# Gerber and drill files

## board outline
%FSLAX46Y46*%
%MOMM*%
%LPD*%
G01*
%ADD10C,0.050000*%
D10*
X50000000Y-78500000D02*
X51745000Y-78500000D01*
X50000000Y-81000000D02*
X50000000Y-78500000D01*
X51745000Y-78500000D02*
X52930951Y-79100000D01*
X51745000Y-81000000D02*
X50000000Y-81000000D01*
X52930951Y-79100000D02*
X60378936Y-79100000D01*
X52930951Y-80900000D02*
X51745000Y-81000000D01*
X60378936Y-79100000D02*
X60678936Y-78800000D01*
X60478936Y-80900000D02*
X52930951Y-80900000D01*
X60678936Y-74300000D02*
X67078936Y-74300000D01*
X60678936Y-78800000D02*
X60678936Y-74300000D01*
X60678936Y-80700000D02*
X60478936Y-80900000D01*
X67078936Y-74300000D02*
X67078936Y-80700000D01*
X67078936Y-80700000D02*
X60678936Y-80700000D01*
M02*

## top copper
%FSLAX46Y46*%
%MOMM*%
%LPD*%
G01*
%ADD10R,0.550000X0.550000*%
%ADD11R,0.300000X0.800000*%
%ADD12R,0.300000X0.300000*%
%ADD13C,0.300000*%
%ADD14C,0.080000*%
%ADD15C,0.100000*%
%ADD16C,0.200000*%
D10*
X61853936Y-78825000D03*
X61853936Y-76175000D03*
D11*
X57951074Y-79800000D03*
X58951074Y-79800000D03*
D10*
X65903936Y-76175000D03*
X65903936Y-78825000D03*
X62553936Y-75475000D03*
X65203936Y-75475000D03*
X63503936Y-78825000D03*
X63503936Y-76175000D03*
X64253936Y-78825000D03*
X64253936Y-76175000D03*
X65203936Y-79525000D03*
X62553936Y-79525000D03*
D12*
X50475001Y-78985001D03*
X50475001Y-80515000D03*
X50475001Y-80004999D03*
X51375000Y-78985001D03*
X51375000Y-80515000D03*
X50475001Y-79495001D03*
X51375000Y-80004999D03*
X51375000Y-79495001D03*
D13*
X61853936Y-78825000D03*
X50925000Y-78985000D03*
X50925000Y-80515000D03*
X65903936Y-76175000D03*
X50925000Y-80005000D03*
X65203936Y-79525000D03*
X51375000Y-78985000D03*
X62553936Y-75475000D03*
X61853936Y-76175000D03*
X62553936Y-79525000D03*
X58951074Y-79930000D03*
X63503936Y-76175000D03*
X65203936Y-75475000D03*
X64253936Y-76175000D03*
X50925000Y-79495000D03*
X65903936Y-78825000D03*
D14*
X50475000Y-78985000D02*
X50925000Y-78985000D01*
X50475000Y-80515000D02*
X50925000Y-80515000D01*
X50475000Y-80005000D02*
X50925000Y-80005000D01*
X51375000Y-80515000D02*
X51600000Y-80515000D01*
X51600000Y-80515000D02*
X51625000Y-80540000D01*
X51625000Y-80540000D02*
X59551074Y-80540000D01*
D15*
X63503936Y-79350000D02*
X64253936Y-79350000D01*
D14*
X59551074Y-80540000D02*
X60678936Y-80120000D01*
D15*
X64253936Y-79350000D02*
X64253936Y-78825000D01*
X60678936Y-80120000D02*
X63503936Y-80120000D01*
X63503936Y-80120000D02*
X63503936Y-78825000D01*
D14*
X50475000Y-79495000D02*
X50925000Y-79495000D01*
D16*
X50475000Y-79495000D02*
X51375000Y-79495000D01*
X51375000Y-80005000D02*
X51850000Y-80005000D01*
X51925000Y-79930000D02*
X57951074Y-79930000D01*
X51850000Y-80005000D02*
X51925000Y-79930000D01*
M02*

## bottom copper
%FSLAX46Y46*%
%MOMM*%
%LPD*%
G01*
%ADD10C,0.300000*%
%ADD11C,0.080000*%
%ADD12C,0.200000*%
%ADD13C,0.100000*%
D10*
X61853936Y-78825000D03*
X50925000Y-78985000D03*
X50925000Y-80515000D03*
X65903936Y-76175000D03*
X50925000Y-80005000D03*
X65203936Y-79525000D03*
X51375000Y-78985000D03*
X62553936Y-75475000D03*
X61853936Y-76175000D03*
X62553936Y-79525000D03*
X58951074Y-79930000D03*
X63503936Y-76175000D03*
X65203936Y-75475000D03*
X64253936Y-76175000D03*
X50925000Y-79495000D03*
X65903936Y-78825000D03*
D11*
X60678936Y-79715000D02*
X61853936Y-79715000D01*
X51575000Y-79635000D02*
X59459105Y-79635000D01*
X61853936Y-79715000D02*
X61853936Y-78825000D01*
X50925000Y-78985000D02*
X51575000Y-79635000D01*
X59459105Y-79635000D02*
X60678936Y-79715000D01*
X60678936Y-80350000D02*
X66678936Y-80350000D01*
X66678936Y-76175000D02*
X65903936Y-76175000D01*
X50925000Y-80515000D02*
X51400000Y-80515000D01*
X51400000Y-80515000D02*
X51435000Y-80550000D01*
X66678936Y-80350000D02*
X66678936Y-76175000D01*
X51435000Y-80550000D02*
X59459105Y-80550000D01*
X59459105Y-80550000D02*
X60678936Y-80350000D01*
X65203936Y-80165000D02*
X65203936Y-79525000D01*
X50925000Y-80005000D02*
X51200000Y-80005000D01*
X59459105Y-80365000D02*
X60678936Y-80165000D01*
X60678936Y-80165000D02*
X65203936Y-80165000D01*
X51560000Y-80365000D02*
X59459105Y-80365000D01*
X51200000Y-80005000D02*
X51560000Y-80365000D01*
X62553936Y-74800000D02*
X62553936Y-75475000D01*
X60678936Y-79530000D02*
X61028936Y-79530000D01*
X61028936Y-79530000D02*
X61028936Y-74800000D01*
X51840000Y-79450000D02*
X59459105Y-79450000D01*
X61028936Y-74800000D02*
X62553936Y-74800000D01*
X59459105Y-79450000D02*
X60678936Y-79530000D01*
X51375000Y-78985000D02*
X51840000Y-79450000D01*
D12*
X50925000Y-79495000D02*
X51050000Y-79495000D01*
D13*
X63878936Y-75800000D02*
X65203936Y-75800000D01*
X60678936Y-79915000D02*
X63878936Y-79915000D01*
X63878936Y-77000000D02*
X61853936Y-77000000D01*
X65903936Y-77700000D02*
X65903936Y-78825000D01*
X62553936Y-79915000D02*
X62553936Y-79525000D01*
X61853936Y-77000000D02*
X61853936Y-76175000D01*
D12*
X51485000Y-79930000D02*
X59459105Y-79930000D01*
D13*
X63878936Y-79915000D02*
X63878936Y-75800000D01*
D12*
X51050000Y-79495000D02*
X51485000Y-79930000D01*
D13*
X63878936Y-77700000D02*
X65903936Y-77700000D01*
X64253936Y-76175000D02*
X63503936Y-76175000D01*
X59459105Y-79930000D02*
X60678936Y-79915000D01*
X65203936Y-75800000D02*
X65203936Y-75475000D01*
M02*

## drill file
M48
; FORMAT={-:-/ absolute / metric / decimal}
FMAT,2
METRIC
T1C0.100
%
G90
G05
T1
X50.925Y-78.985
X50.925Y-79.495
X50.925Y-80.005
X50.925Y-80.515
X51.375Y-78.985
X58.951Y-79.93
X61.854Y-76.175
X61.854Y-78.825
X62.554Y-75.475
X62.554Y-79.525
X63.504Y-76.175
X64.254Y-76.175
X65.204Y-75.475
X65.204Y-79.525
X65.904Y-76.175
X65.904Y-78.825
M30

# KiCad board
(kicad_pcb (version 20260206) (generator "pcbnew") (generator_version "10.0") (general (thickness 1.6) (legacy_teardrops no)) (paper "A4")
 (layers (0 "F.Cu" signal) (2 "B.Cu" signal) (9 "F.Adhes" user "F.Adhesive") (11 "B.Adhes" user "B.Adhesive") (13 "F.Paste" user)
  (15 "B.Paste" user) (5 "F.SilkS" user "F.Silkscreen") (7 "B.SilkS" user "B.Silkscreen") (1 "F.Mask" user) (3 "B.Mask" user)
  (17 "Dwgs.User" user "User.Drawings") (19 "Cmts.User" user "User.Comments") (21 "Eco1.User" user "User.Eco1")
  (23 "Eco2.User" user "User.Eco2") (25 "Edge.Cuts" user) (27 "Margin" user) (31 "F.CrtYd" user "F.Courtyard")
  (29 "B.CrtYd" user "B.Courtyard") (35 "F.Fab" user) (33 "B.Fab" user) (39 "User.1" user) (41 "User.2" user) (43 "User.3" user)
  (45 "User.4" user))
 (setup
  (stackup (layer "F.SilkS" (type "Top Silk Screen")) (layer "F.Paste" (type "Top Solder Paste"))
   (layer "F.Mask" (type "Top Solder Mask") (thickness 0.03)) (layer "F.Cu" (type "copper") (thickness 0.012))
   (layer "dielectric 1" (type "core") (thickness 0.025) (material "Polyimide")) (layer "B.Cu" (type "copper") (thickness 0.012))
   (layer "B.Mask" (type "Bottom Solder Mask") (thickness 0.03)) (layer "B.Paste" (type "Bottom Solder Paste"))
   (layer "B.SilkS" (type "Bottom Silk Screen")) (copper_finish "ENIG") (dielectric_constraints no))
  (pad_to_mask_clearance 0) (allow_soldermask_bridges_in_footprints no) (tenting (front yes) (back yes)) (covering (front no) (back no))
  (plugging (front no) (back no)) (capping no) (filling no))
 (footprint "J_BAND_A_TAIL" (layer "F.Cu") (at 50.9 79.75)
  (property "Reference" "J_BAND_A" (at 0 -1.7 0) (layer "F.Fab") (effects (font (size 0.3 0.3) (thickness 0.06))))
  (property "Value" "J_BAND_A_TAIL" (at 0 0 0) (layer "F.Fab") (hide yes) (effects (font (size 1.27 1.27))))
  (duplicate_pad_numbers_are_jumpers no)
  (pad "1" smd rect (at -0.424999 -0.764999) (size 0.3 0.3) (layers "F.Cu" "F.Mask") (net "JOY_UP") (solder_mask_margin 0.05)
   (thermal_bridge_angle 45))
  (pad "2" smd rect (at -0.424999 0.765) (size 0.3 0.3) (layers "F.Cu" "F.Mask") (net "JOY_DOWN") (solder_mask_margin 0.05)
   (thermal_bridge_angle 45))
  (pad "3" smd rect (at -0.424999 0.254999) (size 0.3 0.3) (layers "F.Cu" "F.Mask") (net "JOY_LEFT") (solder_mask_margin 0.05)
   (thermal_bridge_angle 45))
  (pad "4" smd rect (at 0.475 -0.764999) (size 0.3 0.3) (layers "F.Cu" "F.Mask") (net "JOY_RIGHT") (solder_mask_margin 0.05)
   (thermal_bridge_angle 45))
  (pad "5" smd rect (at 0.475 0.765) (size 0.3 0.3) (layers "F.Cu" "F.Mask") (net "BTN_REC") (solder_mask_margin 0.05)
   (thermal_bridge_angle 45))
  (pad "6" smd rect (at -0.424999 -0.254999) (size 0.3 0.3) (layers "F.Cu" "F.Mask") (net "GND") (solder_mask_margin 0.05)
   (thermal_bridge_angle 45))
  (pad "7" smd rect (at 0.475 0.254999) (size 0.3 0.3) (layers "F.Cu" "F.Mask") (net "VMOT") (solder_mask_margin 0.05)
   (thermal_bridge_angle 45))
  (pad "8" smd rect (at 0.475 -0.254999) (size 0.3 0.3) (layers "F.Cu" "F.Mask") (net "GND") (solder_mask_margin 0.05)
   (thermal_bridge_angle 45)))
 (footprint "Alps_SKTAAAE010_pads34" (layer "F.Cu") (at 61.478936 77.5 90)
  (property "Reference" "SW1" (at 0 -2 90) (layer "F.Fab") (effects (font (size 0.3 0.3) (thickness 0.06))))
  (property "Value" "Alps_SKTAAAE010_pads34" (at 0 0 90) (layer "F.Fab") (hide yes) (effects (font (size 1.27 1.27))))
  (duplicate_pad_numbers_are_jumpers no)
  (pad "3" smd rect (at -1.325 0.375 90) (size 0.55 0.55) (layers "F.Cu" "F.Mask" "F.Paste") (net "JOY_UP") (solder_mask_margin 0.05)
   (thermal_bridge_angle 45))
  (pad "4" smd rect (at 1.325 0.375 90) (size 0.55 0.55) (layers "F.Cu" "F.Mask" "F.Paste") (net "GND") (solder_mask_margin 0.05)
   (thermal_bridge_angle 45)))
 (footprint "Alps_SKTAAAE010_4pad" (layer "F.Cu") (at 63.878936 77.5 90)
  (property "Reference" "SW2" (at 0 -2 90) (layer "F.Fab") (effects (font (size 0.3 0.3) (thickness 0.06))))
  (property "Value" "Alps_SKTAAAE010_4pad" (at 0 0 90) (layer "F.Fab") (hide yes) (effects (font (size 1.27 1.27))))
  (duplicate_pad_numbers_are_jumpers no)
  (pad "1" smd rect (at -1.325 -0.375 90) (size 0.55 0.55) (layers "F.Cu" "F.Mask" "F.Paste") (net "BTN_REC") (solder_mask_margin 0.05)
   (thermal_bridge_angle 45))
  (pad "2" smd rect (at 1.325 -0.375 90) (size 0.55 0.55) (layers "F.Cu" "F.Mask" "F.Paste") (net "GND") (solder_mask_margin 0.05)
   (thermal_bridge_angle 45))
  (pad "3" smd rect (at -1.325 0.375 90) (size 0.55 0.55) (layers "F.Cu" "F.Mask" "F.Paste") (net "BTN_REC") (solder_mask_margin 0.05)
   (thermal_bridge_angle 45))
  (pad "4" smd rect (at 1.325 0.375 90) (size 0.55 0.55) (layers "F.Cu" "F.Mask" "F.Paste") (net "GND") (solder_mask_margin 0.05)
   (thermal_bridge_angle 45)))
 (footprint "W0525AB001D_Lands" (layer "F.Cu") (at 58.451074 79.93)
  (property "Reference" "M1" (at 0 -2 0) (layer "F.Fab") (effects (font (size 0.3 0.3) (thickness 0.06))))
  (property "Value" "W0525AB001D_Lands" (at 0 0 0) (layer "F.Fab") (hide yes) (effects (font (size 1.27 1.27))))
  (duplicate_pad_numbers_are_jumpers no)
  (pad "1" smd rect (at -0.5 -0.13) (size 0.3 0.8) (layers "F.Cu" "F.Mask") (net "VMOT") (solder_mask_margin 0.05) (thermal_bridge_angle 45))
  (pad "2" smd rect (at 0.5 -0.13) (size 0.3 0.8) (layers "F.Cu" "F.Mask") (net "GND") (solder_mask_margin 0.05) (thermal_bridge_angle 45)))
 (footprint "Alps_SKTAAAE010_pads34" (layer "F.Cu") (at 66.278936 77.5 -90)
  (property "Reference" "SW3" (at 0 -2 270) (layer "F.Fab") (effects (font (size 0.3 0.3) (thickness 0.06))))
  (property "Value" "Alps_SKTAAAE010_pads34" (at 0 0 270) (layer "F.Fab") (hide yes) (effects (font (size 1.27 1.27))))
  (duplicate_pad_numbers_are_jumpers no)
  (pad "3" smd rect (at -1.325 0.375 270) (size 0.55 0.55) (layers "F.Cu" "F.Mask" "F.Paste") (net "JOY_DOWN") (solder_mask_margin 0.05)
   (thermal_bridge_angle 45))
  (pad "4" smd rect (at 1.325 0.375 270) (size 0.55 0.55) (layers "F.Cu" "F.Mask" "F.Paste") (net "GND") (solder_mask_margin 0.05)
   (thermal_bridge_angle 45)))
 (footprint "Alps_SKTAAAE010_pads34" (layer "F.Cu") (at 63.878936 79.9 180)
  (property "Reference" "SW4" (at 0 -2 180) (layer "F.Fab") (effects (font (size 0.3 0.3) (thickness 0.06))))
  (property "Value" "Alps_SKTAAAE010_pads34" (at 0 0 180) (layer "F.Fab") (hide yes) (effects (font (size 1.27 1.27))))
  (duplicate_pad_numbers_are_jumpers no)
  (pad "3" smd rect (at -1.325 0.375 180) (size 0.55 0.55) (layers "F.Cu" "F.Mask" "F.Paste") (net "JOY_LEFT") (solder_mask_margin 0.05)
   (thermal_bridge_angle 45))
  (pad "4" smd rect (at 1.325 0.375 180) (size 0.55 0.55) (layers "F.Cu" "F.Mask" "F.Paste") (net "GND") (solder_mask_margin 0.05)
   (thermal_bridge_angle 45)))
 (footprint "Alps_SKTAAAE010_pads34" (layer "F.Cu") (at 63.878936 75.1)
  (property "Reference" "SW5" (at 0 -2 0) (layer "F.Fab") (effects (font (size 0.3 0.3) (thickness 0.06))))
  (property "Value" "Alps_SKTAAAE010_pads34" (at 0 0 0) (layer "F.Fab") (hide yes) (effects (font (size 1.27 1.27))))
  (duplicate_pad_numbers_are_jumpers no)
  (pad "3" smd rect (at -1.325 0.375) (size 0.55 0.55) (layers "F.Cu" "F.Mask" "F.Paste") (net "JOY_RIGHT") (solder_mask_margin 0.05)
   (thermal_bridge_angle 45))
  (pad "4" smd rect (at 1.325 0.375) (size 0.55 0.55) (layers "F.Cu" "F.Mask" "F.Paste") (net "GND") (solder_mask_margin 0.05)
   (thermal_bridge_angle 45)))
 (gr_line (start 50 78.5) (end 51.745 78.5) (stroke (width 0.05) (type default)) (layer "Edge.Cuts"))
 (gr_line (start 50 81) (end 50 78.5) (stroke (width 0.05) (type default)) (layer "Edge.Cuts"))
 (gr_line (start 51.745 78.5) (end 52.930951 79.1) (stroke (width 0.05) (type default)) (layer "Edge.Cuts"))
 (gr_line (start 51.745 81) (end 50 81) (stroke (width 0.05) (type default)) (layer "Edge.Cuts"))
 (gr_line (start 52.930951 79.1) (end 60.378936 79.1) (stroke (width 0.05) (type default)) (layer "Edge.Cuts"))
 (gr_line (start 52.930951 80.9) (end 51.745 81) (stroke (width 0.05) (type default)) (layer "Edge.Cuts"))
 (gr_line (start 60.378936 79.1) (end 60.678936 78.8) (stroke (width 0.05) (type default)) (layer "Edge.Cuts"))
 (gr_line (start 60.478936 80.9) (end 52.930951 80.9) (stroke (width 0.05) (type default)) (layer "Edge.Cuts"))
 (gr_line (start 60.678936 74.3) (end 67.078936 74.3) (stroke (width 0.05) (type default)) (layer "Edge.Cuts"))
 (gr_line (start 60.678936 78.8) (end 60.678936 74.3) (stroke (width 0.05) (type default)) (layer "Edge.Cuts"))
 (gr_line (start 60.678936 80.7) (end 60.478936 80.9) (stroke (width 0.05) (type default)) (layer "Edge.Cuts"))
 (gr_line (start 67.078936 74.3) (end 67.078936 80.7) (stroke (width 0.05) (type default)) (layer "Edge.Cuts"))
 (gr_line (start 67.078936 80.7) (end 60.678936 80.7) (stroke (width 0.05) (type default)) (layer "Edge.Cuts"))
 (segment (start 50.475 78.985) (end 50.925 78.985) (width 0.08) (layer "F.Cu") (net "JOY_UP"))
 (via (at 61.853936 78.825) (size 0.3) (drill 0.1) (layers "F.Cu" "B.Cu") (tenting (front yes) (back yes)) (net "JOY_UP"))
 (via (at 50.925 78.985) (size 0.3) (drill 0.1) (layers "F.Cu" "B.Cu") (tenting (front yes) (back yes)) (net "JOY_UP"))
 (segment (start 60.678936 79.715) (end 61.853936 79.715) (width 0.08) (layer "B.Cu") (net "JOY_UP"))
 (segment (start 61.853936 79.715) (end 61.853936 78.825) (width 0.08) (layer "B.Cu") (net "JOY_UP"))
 (segment (start 59.459105 79.635) (end 60.678936 79.715) (width 0.08) (layer "B.Cu") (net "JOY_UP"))
 (segment (start 51.575 79.635) (end 59.459105 79.635) (width 0.08) (layer "B.Cu") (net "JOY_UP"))
 (segment (start 50.925 78.985) (end 51.575 79.635) (width 0.08) (layer "B.Cu") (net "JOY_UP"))
 (segment (start 50.475 80.515) (end 50.925 80.515) (width 0.08) (layer "F.Cu") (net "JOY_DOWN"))
 (via (at 50.925 80.515) (size 0.3) (drill 0.1) (layers "F.Cu" "B.Cu") (tenting (front yes) (back yes)) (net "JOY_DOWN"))
 (via (at 65.903936 76.175) (size 0.3) (drill 0.1) (layers "F.Cu" "B.Cu") (tenting (front yes) (back yes)) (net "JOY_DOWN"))
 (segment (start 66.678936 80.35) (end 66.678936 76.175) (width 0.08) (layer "B.Cu") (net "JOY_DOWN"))
 (segment (start 66.678936 76.175) (end 65.903936 76.175) (width 0.08) (layer "B.Cu") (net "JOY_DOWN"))
 (segment (start 60.678936 80.35) (end 66.678936 80.35) (width 0.08) (layer "B.Cu") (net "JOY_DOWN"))
 (segment (start 59.459105 80.55) (end 60.678936 80.35) (width 0.08) (layer "B.Cu") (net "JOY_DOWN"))
 (segment (start 51.435 80.55) (end 59.459105 80.55) (width 0.08) (layer "B.Cu") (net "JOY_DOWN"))
 (segment (start 51.4 80.515) (end 51.435 80.55) (width 0.08) (layer "B.Cu") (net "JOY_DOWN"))
 (segment (start 50.925 80.515) (end 51.4 80.515) (width 0.08) (layer "B.Cu") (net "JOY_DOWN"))
 (segment (start 50.475 80.005) (end 50.925 80.005) (width 0.08) (layer "F.Cu") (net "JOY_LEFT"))
 (via (at 65.203936 79.525) (size 0.3) (drill 0.1) (layers "F.Cu" "B.Cu") (tenting (front yes) (back yes)) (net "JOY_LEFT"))
 (via (at 50.925 80.005) (size 0.3) (drill 0.1) (layers "F.Cu" "B.Cu") (tenting (front yes) (back yes)) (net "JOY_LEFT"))
 (segment (start 51.56 80.365) (end 59.459105 80.365) (width 0.08) (layer "B.Cu") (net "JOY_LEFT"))
 (segment (start 65.203936 80.165) (end 65.203936 79.525) (width 0.08) (layer "B.Cu") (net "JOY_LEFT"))
 (segment (start 60.678936 80.165) (end 65.203936 80.165) (width 0.08) (layer "B.Cu") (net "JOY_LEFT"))
 (segment (start 59.459105 80.365) (end 60.678936 80.165) (width 0.08) (layer "B.Cu") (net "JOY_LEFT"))
 (segment (start 51.2 80.005) (end 51.56 80.365) (width 0.08) (layer "B.Cu") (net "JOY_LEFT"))
 (segment (start 50.925 80.005) (end 51.2 80.005) (width 0.08) (layer "B.Cu") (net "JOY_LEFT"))
 (via (at 51.375 78.985) (size 0.3) (drill 0.1) (layers "F.Cu" "B.Cu") (tenting (front yes) (back yes)) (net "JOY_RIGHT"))
 (via (at 62.553936 75.475) (size 0.3) (drill 0.1) (layers "F.Cu" "B.Cu") (tenting (front yes) (back yes)) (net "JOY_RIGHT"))
 (segment (start 51.375 78.985) (end 51.84 79.45) (width 0.08) (layer "B.Cu") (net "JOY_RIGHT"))
 (segment (start 62.553936 74.8) (end 62.553936 75.475) (width 0.08) (layer "B.Cu") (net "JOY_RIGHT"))
 (segment (start 51.84 79.45) (end 59.459105 79.45) (width 0.08) (layer "B.Cu") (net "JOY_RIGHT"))
 (segment (start 60.678936 79.53) (end 61.028936 79.53) (width 0.08) (layer "B.Cu") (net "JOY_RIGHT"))
 (segment (start 61.028936 79.53) (end 61.028936 74.8) (width 0.08) (layer "B.Cu") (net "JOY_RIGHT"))
 (segment (start 59.459105 79.45) (end 60.678936 79.53) (width 0.08) (layer "B.Cu") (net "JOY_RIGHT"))
 (segment (start 61.028936 74.8) (end 62.553936 74.8) (width 0.08) (layer "B.Cu") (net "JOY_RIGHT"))
 (segment (start 59.551074 80.54) (end 60.678936 80.12) (width 0.08) (layer "F.Cu") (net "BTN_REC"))
 (segment (start 63.503936 79.35) (end 64.253936 79.35) (width 0.1) (layer "F.Cu") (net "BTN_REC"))
 (segment (start 60.678936 80.12) (end 63.503936 80.12) (width 0.1) (layer "F.Cu") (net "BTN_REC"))
 (segment (start 51.375 80.515) (end 51.6 80.515) (width 0.08) (layer "F.Cu") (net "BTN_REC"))
 (segment (start 63.503936 80.12) (end 63.503936 78.825) (width 0.1) (layer "F.Cu") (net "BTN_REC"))
 (segment (start 64.253936 79.35) (end 64.253936 78.825) (width 0.1) (layer "F.Cu") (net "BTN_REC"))
 (segment (start 51.625 80.54) (end 59.551074 80.54) (width 0.08) (layer "F.Cu") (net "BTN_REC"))
 (segment (start 51.6 80.515) (end 51.625 80.54) (width 0.08) (layer "F.Cu") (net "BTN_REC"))
 (segment (start 50.475 79.495) (end 50.925 79.495) (width 0.08) (layer "F.Cu") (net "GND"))
 (segment (start 50.475 79.495) (end 51.375 79.495) (width 0.2) (layer "F.Cu") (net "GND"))
 (via (at 63.503936 76.175) (size 0.3) (drill 0.1) (layers "F.Cu" "B.Cu") (tenting (front yes) (back yes)) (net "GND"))
 (via (at 61.853936 76.175) (size 0.3) (drill 0.1) (layers "F.Cu" "B.Cu") (tenting (front yes) (back yes)) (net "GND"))
 (via (at 62.553936 79.525) (size 0.3) (drill 0.1) (layers "F.Cu" "B.Cu") (tenting (front yes) (back yes)) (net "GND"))
 (via (at 58.951074 79.93) (size 0.3) (drill 0.1) (layers "F.Cu" "B.Cu") (tenting (front yes) (back yes)) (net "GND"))
 (via (at 65.903936 78.825) (size 0.3) (drill 0.1) (layers "F.Cu" "B.Cu") (tenting (front yes) (back yes)) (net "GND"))
 (via (at 50.925 79.495) (size 0.3) (drill 0.1) (layers "F.Cu" "B.Cu") (tenting (front yes) (back yes)) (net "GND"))
 (via (at 65.203936 75.475) (size 0.3) (drill 0.1) (layers "F.Cu" "B.Cu") (tenting (front yes) (back yes)) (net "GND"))
 (via (at 64.253936 76.175) (size 0.3) (drill 0.1) (layers "F.Cu" "B.Cu") (tenting (front yes) (back yes)) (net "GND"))
 (segment (start 65.903936 77.7) (end 65.903936 78.825) (width 0.1) (layer "B.Cu") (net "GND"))
 (segment (start 51.05 79.495) (end 51.485 79.93) (width 0.2) (layer "B.Cu") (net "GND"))
 (segment (start 50.925 79.495) (end 51.05 79.495) (width 0.2) (layer "B.Cu") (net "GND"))
 (segment (start 63.878936 75.8) (end 65.203936 75.8) (width 0.1) (layer "B.Cu") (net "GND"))
 (segment (start 65.203936 75.8) (end 65.203936 75.475) (width 0.1) (layer "B.Cu") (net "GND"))
 (segment (start 60.678936 79.915) (end 63.878936 79.915) (width 0.1) (layer "B.Cu") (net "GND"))
 (segment (start 63.878936 79.915) (end 63.878936 75.8) (width 0.1) (layer "B.Cu") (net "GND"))
 (segment (start 63.878936 77) (end 61.853936 77) (width 0.1) (layer "B.Cu") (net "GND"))
 (segment (start 64.253936 76.175) (end 63.503936 76.175) (width 0.1) (layer "B.Cu") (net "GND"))
 (segment (start 62.553936 79.915) (end 62.553936 79.525) (width 0.1) (layer "B.Cu") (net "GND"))
 (segment (start 59.459105 79.93) (end 60.678936 79.915) (width 0.1) (layer "B.Cu") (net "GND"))
 (segment (start 61.853936 77) (end 61.853936 76.175) (width 0.1) (layer "B.Cu") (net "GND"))
 (segment (start 51.485 79.93) (end 59.459105 79.93) (width 0.2) (layer "B.Cu") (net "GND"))
 (segment (start 63.878936 77.7) (end 65.903936 77.7) (width 0.1) (layer "B.Cu") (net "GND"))
 (segment (start 51.375 80.005) (end 51.85 80.005) (width 0.2) (layer "F.Cu") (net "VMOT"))
 (segment (start 51.85 80.005) (end 51.925 79.93) (width 0.2) (layer "F.Cu") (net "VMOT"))
 (segment (start 51.925 79.93) (end 57.951074 79.93) (width 0.2) (layer "F.Cu") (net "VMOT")))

